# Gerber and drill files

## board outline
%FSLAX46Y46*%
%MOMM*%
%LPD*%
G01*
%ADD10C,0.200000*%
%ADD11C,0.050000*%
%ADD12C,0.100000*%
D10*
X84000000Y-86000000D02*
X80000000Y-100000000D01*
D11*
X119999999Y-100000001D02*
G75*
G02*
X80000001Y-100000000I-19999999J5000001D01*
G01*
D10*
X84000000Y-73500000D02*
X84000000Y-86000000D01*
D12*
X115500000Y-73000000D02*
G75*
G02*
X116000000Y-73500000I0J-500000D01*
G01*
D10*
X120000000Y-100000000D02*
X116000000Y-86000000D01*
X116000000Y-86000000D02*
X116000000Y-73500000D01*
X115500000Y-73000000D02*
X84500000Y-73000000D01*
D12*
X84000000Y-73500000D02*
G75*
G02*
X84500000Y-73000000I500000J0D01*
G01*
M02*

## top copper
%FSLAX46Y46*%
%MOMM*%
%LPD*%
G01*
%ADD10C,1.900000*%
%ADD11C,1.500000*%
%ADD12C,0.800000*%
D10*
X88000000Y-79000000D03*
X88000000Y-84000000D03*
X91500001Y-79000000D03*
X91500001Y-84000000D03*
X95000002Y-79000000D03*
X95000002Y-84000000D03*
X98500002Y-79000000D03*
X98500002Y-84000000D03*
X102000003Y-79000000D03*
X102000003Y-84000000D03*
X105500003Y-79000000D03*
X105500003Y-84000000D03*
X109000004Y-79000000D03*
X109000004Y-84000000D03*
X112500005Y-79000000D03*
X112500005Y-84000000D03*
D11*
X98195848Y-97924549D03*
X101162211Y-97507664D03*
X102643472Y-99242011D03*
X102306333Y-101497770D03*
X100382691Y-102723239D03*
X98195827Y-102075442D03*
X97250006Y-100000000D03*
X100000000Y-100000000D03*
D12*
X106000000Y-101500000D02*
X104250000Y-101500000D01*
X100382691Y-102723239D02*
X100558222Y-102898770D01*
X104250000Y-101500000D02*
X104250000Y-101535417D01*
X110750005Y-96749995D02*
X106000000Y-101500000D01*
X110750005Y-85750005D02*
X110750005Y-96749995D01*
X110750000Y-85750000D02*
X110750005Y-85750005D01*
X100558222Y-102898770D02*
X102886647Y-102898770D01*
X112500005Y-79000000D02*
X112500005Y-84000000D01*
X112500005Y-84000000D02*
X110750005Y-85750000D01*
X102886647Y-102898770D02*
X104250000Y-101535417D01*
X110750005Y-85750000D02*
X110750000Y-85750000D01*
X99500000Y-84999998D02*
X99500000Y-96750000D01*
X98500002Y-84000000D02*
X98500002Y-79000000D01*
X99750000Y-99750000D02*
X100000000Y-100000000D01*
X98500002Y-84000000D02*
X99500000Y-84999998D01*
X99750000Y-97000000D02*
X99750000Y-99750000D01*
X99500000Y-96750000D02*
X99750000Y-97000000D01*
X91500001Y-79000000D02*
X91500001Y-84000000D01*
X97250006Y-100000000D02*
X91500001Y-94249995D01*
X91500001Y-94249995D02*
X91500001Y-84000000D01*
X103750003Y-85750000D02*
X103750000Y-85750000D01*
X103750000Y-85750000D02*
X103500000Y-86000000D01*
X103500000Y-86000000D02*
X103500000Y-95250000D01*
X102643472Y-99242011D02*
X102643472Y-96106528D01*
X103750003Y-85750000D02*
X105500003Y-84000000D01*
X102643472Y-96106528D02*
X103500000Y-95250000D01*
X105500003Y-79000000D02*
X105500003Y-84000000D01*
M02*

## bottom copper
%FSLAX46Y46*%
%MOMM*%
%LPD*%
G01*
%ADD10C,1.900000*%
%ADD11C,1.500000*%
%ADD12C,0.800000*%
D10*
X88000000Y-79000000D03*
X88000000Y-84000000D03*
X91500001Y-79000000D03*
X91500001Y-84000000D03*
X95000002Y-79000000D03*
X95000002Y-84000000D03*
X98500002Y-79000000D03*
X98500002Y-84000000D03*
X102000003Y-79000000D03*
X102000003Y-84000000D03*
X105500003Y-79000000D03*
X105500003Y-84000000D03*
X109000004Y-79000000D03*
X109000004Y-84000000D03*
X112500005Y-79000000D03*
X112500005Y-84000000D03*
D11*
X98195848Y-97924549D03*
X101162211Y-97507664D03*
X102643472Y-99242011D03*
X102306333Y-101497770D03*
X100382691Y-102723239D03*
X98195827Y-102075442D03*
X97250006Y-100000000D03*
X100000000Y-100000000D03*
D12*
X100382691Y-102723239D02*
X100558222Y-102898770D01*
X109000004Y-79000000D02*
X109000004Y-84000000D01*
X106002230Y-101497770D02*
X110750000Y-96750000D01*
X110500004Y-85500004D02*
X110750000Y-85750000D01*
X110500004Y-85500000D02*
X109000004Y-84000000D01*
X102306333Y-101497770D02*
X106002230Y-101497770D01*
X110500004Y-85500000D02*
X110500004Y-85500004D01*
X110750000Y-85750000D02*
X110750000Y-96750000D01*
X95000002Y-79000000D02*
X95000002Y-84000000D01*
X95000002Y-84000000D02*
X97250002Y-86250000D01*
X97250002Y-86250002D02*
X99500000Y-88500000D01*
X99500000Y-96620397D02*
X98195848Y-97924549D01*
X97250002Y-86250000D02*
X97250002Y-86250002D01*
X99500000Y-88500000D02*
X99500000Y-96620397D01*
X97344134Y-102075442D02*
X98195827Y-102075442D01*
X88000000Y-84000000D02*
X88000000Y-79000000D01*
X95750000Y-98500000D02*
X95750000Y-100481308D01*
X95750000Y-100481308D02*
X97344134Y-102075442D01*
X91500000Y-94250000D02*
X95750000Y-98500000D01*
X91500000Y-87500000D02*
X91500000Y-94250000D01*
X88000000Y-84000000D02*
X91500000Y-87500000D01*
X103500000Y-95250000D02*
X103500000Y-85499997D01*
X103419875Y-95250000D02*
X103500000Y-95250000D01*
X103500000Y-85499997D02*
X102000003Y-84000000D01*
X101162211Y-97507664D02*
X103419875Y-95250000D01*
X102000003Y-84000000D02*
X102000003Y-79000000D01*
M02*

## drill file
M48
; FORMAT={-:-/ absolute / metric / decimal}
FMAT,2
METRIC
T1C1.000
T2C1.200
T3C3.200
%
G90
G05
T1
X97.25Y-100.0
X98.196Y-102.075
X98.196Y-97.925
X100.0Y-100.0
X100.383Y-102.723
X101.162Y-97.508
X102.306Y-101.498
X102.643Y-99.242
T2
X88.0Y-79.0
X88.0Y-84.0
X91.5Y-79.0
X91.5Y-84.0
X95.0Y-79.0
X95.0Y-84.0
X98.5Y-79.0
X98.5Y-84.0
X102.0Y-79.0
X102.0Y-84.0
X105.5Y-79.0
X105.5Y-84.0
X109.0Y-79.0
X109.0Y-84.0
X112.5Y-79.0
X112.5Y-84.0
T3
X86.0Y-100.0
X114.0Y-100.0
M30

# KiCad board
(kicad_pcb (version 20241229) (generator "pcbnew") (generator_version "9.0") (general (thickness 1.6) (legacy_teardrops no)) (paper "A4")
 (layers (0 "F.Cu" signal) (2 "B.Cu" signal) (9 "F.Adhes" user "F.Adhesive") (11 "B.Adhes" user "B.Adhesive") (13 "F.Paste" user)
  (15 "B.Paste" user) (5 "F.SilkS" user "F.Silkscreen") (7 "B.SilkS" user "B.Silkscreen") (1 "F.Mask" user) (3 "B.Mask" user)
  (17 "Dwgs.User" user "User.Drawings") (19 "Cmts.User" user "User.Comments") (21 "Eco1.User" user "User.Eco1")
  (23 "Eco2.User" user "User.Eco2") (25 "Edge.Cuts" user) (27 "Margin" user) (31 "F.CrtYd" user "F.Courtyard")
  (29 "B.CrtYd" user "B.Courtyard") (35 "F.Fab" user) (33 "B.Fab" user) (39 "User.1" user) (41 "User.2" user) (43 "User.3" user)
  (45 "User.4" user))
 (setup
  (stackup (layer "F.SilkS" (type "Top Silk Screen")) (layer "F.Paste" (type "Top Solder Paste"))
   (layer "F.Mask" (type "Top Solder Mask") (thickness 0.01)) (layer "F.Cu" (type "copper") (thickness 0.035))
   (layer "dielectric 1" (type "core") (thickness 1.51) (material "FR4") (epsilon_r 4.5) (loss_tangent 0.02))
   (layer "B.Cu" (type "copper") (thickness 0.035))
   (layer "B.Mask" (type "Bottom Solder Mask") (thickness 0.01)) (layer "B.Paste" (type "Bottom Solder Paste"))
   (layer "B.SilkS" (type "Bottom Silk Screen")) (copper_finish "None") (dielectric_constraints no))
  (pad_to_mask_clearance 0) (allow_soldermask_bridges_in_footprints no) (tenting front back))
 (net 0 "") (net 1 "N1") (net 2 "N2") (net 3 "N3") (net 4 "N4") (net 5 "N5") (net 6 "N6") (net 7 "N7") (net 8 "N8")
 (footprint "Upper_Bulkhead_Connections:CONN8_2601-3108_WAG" (layer "F.Cu") (at 88 79)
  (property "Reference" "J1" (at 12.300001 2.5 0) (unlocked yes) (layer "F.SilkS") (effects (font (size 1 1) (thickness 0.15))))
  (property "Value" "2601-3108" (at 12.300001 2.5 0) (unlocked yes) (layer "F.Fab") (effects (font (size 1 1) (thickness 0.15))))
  (pad "1" thru_hole circle (at 0 0) (size 1.9 1.9) (drill 1.2) (layers "*.Cu" "*.Mask") (remove_unused_layers no) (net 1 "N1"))
  (pad "2" thru_hole circle (at 0 5) (size 1.9 1.9) (drill 1.2) (layers "*.Cu" "*.Mask") (remove_unused_layers no) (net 1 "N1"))
  (pad "3" thru_hole circle (at 3.500001 0) (size 1.9 1.9) (drill 1.2) (layers "*.Cu" "*.Mask") (remove_unused_layers no) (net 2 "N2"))
  (pad "4" thru_hole circle (at 3.500001 5) (size 1.9 1.9) (drill 1.2) (layers "*.Cu" "*.Mask") (remove_unused_layers no) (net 2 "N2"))
  (pad "5" thru_hole circle (at 7.000002 0) (size 1.9 1.9) (drill 1.2) (layers "*.Cu" "*.Mask") (remove_unused_layers no) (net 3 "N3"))
  (pad "6" thru_hole circle (at 7.000002 5) (size 1.9 1.9) (drill 1.2) (layers "*.Cu" "*.Mask") (remove_unused_layers no) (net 3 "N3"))
  (pad "7" thru_hole circle (at 10.500002 0) (size 1.9 1.9) (drill 1.2) (layers "*.Cu" "*.Mask") (remove_unused_layers no) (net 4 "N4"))
  (pad "8" thru_hole circle (at 10.500002 5) (size 1.9 1.9) (drill 1.2) (layers "*.Cu" "*.Mask") (remove_unused_layers no) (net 4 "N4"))
  (pad "9" thru_hole circle (at 14.000003 0) (size 1.9 1.9) (drill 1.2) (layers "*.Cu" "*.Mask") (remove_unused_layers no) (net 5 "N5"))
  (pad "10" thru_hole circle (at 14.000003 5) (size 1.9 1.9) (drill 1.2) (layers "*.Cu" "*.Mask") (remove_unused_layers no) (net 5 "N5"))
  (pad "11" thru_hole circle (at 17.500003 0) (size 1.9 1.9) (drill 1.2) (layers "*.Cu" "*.Mask") (remove_unused_layers no) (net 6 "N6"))
  (pad "12" thru_hole circle (at 17.500003 5) (size 1.9 1.9) (drill 1.2) (layers "*.Cu" "*.Mask") (remove_unused_layers no) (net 6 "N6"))
  (pad "13" thru_hole circle (at 21.000004 0) (size 1.9 1.9) (drill 1.2) (layers "*.Cu" "*.Mask") (remove_unused_layers no) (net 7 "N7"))
  (pad "14" thru_hole circle (at 21.000004 5) (size 1.9 1.9) (drill 1.2) (layers "*.Cu" "*.Mask") (remove_unused_layers no) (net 7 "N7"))
  (pad "15" thru_hole circle (at 24.500005 0) (size 1.9 1.9) (drill 1.2) (layers "*.Cu" "*.Mask") (remove_unused_layers no) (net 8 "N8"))
  (pad "16" thru_hole circle (at 24.500005 5) (size 1.9 1.9) (drill 1.2) (layers "*.Cu" "*.Mask") (remove_unused_layers no) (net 8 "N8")))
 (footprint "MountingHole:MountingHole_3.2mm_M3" (layer "F.Cu") (at 86 100)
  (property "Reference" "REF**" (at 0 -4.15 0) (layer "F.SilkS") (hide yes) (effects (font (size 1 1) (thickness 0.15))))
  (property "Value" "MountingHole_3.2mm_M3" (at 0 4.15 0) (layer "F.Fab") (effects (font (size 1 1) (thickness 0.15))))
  (pad "" np_thru_hole circle (at 0 0) (size 3.2 3.2) (drill 3.2) (layers "*.Cu" "*.Mask")))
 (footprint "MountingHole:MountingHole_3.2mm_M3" (layer "F.Cu") (at 114 100)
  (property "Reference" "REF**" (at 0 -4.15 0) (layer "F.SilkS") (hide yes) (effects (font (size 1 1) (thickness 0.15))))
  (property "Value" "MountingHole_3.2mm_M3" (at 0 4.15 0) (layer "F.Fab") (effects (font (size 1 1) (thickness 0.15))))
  (pad "" np_thru_hole circle (at 0 0) (size 3.2 3.2) (drill 3.2) (layers "*.Cu" "*.Mask")))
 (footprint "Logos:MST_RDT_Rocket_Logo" (layer "F.Cu") (at 110 107)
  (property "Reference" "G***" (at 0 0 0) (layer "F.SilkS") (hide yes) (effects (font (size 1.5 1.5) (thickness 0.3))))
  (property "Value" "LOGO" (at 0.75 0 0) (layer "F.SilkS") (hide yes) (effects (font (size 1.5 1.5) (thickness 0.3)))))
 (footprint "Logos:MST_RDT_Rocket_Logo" (layer "B.Cu") (at 90 107 180)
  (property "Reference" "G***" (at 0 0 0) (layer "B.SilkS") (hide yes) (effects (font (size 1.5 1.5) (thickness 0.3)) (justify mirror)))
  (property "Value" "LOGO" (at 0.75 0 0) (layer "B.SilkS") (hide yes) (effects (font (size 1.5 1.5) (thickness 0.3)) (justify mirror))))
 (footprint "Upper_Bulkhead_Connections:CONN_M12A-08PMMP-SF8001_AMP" (layer "B.Cu") (at 100 100 90)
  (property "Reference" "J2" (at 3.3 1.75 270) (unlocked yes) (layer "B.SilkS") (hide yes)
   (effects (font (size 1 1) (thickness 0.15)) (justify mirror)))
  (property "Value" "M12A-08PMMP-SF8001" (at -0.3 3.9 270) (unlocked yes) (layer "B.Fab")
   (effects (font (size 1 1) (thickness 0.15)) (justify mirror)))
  (pad "1" thru_hole circle (at 2.075451 -1.804152 90) (size 1.5 1.5) (drill 1) (layers "*.Cu" "*.Mask") (remove_unused_layers no)
   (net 3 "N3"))
  (pad "2" thru_hole circle (at 2.492336 1.162211 38.572) (size 1.5 1.5) (drill 1) (layers "*.Cu" "*.Mask") (remove_unused_layers no)
   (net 5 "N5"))
  (pad "3" thru_hole circle (at 0.757989 2.643472 347.143) (size 1.5 1.5) (drill 1) (layers "*.Cu" "*.Mask") (remove_unused_layers no)
   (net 6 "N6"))
  (pad "4" thru_hole circle (at -1.49777 2.306333 295.715) (size 1.5 1.5) (drill 1) (layers "*.Cu" "*.Mask") (remove_unused_layers no)
   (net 7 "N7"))
  (pad "5" thru_hole circle (at -2.723239 0.382691 244.286) (size 1.5 1.5) (drill 1) (layers "*.Cu" "*.Mask") (remove_unused_layers no)
   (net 8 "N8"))
  (pad "6" thru_hole circle (at -2.075442 -1.804173 192.858) (size 1.5 1.5) (drill 1) (layers "*.Cu" "*.Mask") (remove_unused_layers no)
   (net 1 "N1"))
  (pad "7" thru_hole circle (at 0 -2.749994 141.429) (size 1.5 1.5) (drill 1) (layers "*.Cu" "*.Mask") (remove_unused_layers no)
   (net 2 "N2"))
  (pad "8" thru_hole circle (at 0 0 90) (size 1.5 1.5) (drill 1) (layers "*.Cu" "*.Mask") (remove_unused_layers no) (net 4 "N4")))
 (gr_line (start 84 86) (end 80 100) (stroke (width 0.2) (type solid)) (layer "Edge.Cuts"))
 (gr_arc (start 119.999999 100.000001) (mid 100 115.615527) (end 80.000001 100) (stroke (width 0.05) (type solid)) (layer "Edge.Cuts"))
 (gr_line (start 84 73.5) (end 84 86) (stroke (width 0.2) (type solid)) (layer "Edge.Cuts"))
 (gr_arc (start 115.5 73) (mid 115.853553 73.146447) (end 116 73.5) (stroke (width 0.1) (type solid)) (layer "Edge.Cuts"))
 (gr_line (start 120 100) (end 116 86) (stroke (width 0.2) (type solid)) (layer "Edge.Cuts"))
 (gr_line (start 116 86) (end 116 73.5) (stroke (width 0.2) (type solid)) (layer "Edge.Cuts"))
 (gr_line (start 115.5 73) (end 84.5 73) (stroke (width 0.2) (type solid)) (layer "Edge.Cuts"))
 (gr_arc (start 84 73.5) (mid 84.146447 73.146447) (end 84.5 73) (stroke (width 0.1) (type solid)) (layer "Edge.Cuts"))
 (segment (start 106 101.5) (end 104.25 101.5) (width 0.8) (layer "F.Cu") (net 8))
 (segment (start 100.382691 102.723239) (end 100.558222 102.89877) (width 0.8) (layer "F.Cu") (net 8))
 (segment (start 104.25 101.5) (end 104.25 101.535417) (width 0.8) (layer "F.Cu") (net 8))
 (segment (start 110.750005 96.749995) (end 106 101.5) (width 0.8) (layer "F.Cu") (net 8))
 (segment (start 110.750005 85.750005) (end 110.750005 96.749995) (width 0.8) (layer "F.Cu") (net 8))
 (segment (start 110.75 85.75) (end 110.750005 85.750005) (width 0.8) (layer "F.Cu") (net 8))
 (segment (start 100.558222 102.89877) (end 102.886647 102.89877) (width 0.8) (layer "F.Cu") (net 8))
 (segment (start 112.500005 79) (end 112.500005 84) (width 0.8) (layer "F.Cu") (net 8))
 (segment (start 112.500005 84) (end 110.750005 85.75) (width 0.8) (layer "F.Cu") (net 8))
 (segment (start 102.886647 102.89877) (end 104.25 101.535417) (width 0.8) (layer "F.Cu") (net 8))
 (segment (start 110.750005 85.75) (end 110.75 85.75) (width 0.8) (layer "F.Cu") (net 8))
 (segment (start 100.382691 102.723239) (end 100.558222 102.89877) (width 0.8) (layer "B.Cu") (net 8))
 (segment (start 99.5 84.999998) (end 99.5 96.75) (width 0.8) (layer "F.Cu") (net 4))
 (segment (start 98.500002 84) (end 98.500002 79) (width 0.8) (layer "F.Cu") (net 4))
 (segment (start 99.75 99.75) (end 100 100) (width 0.8) (layer "F.Cu") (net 4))
 (segment (start 98.500002 84) (end 99.5 84.999998) (width 0.8) (layer "F.Cu") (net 4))
 (segment (start 99.75 97) (end 99.75 99.75) (width 0.8) (layer "F.Cu") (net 4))
 (segment (start 99.5 96.75) (end 99.75 97) (width 0.8) (layer "F.Cu") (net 4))
 (segment (start 109.000004 79) (end 109.000004 84) (width 0.8) (layer "B.Cu") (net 7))
 (segment (start 106.00223 101.49777) (end 110.75 96.75) (width 0.8) (layer "B.Cu") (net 7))
 (segment (start 110.500004 85.500004) (end 110.75 85.75) (width 0.8) (layer "B.Cu") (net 7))
 (segment (start 110.500004 85.5) (end 109.000004 84) (width 0.8) (layer "B.Cu") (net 7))
 (segment (start 102.306333 101.49777) (end 106.00223 101.49777) (width 0.8) (layer "B.Cu") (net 7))
 (segment (start 110.500004 85.5) (end 110.500004 85.500004) (width 0.8) (layer "B.Cu") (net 7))
 (segment (start 110.75 85.75) (end 110.75 96.75) (width 0.8) (layer "B.Cu") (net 7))
 (segment (start 91.500001 79) (end 91.500001 84) (width 0.8) (layer "F.Cu") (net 2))
 (segment (start 97.250006 100) (end 91.500001 94.249995) (width 0.8) (layer "F.Cu") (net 2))
 (segment (start 91.500001 94.249995) (end 91.500001 84) (width 0.8) (layer "F.Cu") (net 2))
 (segment (start 103.750003 85.75) (end 103.75 85.75) (width 0.8) (layer "F.Cu") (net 6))
 (segment (start 103.75 85.75) (end 103.5 86) (width 0.8) (layer "F.Cu") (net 6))
 (segment (start 103.5 86) (end 103.5 95.25) (width 0.8) (layer "F.Cu") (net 6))
 (segment (start 102.643472 99.242011) (end 102.643472 96.106528) (width 0.8) (layer "F.Cu") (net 6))
 (segment (start 103.750003 85.75) (end 105.500003 84) (width 0.8) (layer "F.Cu") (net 6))
 (segment (start 102.643472 96.106528) (end 103.5 95.25) (width 0.8) (layer "F.Cu") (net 6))
 (segment (start 105.500003 79) (end 105.500003 84) (width 0.8) (layer "F.Cu") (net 6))
 (segment (start 95.000002 79) (end 95.000002 84) (width 0.8) (layer "B.Cu") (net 3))
 (segment (start 95.000002 84) (end 97.250002 86.25) (width 0.8) (layer "B.Cu") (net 3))
 (segment (start 97.250002 86.250002) (end 99.5 88.5) (width 0.8) (layer "B.Cu") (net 3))
 (segment (start 99.5 96.620397) (end 98.195848 97.924549) (width 0.8) (layer "B.Cu") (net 3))
 (segment (start 97.250002 86.25) (end 97.250002 86.250002) (width 0.8) (layer "B.Cu") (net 3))
 (segment (start 99.5 88.5) (end 99.5 96.620397) (width 0.8) (layer "B.Cu") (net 3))
 (segment (start 97.344134 102.075442) (end 98.195827 102.075442) (width 0.8) (layer "B.Cu") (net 1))
 (segment (start 88 84) (end 88 79) (width 0.8) (layer "B.Cu") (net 1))
 (segment (start 95.75 98.5) (end 95.75 100.481308) (width 0.8) (layer "B.Cu") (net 1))
 (segment (start 95.75 100.481308) (end 97.344134 102.075442) (width 0.8) (layer "B.Cu") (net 1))
 (segment (start 91.5 94.25) (end 95.75 98.5) (width 0.8) (layer "B.Cu") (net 1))
 (segment (start 91.5 87.5) (end 91.5 94.25) (width 0.8) (layer "B.Cu") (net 1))
 (segment (start 88 84) (end 91.5 87.5) (width 0.8) (layer "B.Cu") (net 1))
 (segment (start 103.5 95.25) (end 103.5 85.499997) (width 0.8) (layer "B.Cu") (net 5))
 (segment (start 103.419875 95.25) (end 103.5 95.25) (width 0.8) (layer "B.Cu") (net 5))
 (segment (start 103.5 85.499997) (end 102.000003 84) (width 0.8) (layer "B.Cu") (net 5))
 (segment (start 101.162211 97.507664) (end 103.419875 95.25) (width 0.8) (layer "B.Cu") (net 5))
 (segment (start 102.000003 84) (end 102.000003 79) (width 0.8) (layer "B.Cu") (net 5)))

